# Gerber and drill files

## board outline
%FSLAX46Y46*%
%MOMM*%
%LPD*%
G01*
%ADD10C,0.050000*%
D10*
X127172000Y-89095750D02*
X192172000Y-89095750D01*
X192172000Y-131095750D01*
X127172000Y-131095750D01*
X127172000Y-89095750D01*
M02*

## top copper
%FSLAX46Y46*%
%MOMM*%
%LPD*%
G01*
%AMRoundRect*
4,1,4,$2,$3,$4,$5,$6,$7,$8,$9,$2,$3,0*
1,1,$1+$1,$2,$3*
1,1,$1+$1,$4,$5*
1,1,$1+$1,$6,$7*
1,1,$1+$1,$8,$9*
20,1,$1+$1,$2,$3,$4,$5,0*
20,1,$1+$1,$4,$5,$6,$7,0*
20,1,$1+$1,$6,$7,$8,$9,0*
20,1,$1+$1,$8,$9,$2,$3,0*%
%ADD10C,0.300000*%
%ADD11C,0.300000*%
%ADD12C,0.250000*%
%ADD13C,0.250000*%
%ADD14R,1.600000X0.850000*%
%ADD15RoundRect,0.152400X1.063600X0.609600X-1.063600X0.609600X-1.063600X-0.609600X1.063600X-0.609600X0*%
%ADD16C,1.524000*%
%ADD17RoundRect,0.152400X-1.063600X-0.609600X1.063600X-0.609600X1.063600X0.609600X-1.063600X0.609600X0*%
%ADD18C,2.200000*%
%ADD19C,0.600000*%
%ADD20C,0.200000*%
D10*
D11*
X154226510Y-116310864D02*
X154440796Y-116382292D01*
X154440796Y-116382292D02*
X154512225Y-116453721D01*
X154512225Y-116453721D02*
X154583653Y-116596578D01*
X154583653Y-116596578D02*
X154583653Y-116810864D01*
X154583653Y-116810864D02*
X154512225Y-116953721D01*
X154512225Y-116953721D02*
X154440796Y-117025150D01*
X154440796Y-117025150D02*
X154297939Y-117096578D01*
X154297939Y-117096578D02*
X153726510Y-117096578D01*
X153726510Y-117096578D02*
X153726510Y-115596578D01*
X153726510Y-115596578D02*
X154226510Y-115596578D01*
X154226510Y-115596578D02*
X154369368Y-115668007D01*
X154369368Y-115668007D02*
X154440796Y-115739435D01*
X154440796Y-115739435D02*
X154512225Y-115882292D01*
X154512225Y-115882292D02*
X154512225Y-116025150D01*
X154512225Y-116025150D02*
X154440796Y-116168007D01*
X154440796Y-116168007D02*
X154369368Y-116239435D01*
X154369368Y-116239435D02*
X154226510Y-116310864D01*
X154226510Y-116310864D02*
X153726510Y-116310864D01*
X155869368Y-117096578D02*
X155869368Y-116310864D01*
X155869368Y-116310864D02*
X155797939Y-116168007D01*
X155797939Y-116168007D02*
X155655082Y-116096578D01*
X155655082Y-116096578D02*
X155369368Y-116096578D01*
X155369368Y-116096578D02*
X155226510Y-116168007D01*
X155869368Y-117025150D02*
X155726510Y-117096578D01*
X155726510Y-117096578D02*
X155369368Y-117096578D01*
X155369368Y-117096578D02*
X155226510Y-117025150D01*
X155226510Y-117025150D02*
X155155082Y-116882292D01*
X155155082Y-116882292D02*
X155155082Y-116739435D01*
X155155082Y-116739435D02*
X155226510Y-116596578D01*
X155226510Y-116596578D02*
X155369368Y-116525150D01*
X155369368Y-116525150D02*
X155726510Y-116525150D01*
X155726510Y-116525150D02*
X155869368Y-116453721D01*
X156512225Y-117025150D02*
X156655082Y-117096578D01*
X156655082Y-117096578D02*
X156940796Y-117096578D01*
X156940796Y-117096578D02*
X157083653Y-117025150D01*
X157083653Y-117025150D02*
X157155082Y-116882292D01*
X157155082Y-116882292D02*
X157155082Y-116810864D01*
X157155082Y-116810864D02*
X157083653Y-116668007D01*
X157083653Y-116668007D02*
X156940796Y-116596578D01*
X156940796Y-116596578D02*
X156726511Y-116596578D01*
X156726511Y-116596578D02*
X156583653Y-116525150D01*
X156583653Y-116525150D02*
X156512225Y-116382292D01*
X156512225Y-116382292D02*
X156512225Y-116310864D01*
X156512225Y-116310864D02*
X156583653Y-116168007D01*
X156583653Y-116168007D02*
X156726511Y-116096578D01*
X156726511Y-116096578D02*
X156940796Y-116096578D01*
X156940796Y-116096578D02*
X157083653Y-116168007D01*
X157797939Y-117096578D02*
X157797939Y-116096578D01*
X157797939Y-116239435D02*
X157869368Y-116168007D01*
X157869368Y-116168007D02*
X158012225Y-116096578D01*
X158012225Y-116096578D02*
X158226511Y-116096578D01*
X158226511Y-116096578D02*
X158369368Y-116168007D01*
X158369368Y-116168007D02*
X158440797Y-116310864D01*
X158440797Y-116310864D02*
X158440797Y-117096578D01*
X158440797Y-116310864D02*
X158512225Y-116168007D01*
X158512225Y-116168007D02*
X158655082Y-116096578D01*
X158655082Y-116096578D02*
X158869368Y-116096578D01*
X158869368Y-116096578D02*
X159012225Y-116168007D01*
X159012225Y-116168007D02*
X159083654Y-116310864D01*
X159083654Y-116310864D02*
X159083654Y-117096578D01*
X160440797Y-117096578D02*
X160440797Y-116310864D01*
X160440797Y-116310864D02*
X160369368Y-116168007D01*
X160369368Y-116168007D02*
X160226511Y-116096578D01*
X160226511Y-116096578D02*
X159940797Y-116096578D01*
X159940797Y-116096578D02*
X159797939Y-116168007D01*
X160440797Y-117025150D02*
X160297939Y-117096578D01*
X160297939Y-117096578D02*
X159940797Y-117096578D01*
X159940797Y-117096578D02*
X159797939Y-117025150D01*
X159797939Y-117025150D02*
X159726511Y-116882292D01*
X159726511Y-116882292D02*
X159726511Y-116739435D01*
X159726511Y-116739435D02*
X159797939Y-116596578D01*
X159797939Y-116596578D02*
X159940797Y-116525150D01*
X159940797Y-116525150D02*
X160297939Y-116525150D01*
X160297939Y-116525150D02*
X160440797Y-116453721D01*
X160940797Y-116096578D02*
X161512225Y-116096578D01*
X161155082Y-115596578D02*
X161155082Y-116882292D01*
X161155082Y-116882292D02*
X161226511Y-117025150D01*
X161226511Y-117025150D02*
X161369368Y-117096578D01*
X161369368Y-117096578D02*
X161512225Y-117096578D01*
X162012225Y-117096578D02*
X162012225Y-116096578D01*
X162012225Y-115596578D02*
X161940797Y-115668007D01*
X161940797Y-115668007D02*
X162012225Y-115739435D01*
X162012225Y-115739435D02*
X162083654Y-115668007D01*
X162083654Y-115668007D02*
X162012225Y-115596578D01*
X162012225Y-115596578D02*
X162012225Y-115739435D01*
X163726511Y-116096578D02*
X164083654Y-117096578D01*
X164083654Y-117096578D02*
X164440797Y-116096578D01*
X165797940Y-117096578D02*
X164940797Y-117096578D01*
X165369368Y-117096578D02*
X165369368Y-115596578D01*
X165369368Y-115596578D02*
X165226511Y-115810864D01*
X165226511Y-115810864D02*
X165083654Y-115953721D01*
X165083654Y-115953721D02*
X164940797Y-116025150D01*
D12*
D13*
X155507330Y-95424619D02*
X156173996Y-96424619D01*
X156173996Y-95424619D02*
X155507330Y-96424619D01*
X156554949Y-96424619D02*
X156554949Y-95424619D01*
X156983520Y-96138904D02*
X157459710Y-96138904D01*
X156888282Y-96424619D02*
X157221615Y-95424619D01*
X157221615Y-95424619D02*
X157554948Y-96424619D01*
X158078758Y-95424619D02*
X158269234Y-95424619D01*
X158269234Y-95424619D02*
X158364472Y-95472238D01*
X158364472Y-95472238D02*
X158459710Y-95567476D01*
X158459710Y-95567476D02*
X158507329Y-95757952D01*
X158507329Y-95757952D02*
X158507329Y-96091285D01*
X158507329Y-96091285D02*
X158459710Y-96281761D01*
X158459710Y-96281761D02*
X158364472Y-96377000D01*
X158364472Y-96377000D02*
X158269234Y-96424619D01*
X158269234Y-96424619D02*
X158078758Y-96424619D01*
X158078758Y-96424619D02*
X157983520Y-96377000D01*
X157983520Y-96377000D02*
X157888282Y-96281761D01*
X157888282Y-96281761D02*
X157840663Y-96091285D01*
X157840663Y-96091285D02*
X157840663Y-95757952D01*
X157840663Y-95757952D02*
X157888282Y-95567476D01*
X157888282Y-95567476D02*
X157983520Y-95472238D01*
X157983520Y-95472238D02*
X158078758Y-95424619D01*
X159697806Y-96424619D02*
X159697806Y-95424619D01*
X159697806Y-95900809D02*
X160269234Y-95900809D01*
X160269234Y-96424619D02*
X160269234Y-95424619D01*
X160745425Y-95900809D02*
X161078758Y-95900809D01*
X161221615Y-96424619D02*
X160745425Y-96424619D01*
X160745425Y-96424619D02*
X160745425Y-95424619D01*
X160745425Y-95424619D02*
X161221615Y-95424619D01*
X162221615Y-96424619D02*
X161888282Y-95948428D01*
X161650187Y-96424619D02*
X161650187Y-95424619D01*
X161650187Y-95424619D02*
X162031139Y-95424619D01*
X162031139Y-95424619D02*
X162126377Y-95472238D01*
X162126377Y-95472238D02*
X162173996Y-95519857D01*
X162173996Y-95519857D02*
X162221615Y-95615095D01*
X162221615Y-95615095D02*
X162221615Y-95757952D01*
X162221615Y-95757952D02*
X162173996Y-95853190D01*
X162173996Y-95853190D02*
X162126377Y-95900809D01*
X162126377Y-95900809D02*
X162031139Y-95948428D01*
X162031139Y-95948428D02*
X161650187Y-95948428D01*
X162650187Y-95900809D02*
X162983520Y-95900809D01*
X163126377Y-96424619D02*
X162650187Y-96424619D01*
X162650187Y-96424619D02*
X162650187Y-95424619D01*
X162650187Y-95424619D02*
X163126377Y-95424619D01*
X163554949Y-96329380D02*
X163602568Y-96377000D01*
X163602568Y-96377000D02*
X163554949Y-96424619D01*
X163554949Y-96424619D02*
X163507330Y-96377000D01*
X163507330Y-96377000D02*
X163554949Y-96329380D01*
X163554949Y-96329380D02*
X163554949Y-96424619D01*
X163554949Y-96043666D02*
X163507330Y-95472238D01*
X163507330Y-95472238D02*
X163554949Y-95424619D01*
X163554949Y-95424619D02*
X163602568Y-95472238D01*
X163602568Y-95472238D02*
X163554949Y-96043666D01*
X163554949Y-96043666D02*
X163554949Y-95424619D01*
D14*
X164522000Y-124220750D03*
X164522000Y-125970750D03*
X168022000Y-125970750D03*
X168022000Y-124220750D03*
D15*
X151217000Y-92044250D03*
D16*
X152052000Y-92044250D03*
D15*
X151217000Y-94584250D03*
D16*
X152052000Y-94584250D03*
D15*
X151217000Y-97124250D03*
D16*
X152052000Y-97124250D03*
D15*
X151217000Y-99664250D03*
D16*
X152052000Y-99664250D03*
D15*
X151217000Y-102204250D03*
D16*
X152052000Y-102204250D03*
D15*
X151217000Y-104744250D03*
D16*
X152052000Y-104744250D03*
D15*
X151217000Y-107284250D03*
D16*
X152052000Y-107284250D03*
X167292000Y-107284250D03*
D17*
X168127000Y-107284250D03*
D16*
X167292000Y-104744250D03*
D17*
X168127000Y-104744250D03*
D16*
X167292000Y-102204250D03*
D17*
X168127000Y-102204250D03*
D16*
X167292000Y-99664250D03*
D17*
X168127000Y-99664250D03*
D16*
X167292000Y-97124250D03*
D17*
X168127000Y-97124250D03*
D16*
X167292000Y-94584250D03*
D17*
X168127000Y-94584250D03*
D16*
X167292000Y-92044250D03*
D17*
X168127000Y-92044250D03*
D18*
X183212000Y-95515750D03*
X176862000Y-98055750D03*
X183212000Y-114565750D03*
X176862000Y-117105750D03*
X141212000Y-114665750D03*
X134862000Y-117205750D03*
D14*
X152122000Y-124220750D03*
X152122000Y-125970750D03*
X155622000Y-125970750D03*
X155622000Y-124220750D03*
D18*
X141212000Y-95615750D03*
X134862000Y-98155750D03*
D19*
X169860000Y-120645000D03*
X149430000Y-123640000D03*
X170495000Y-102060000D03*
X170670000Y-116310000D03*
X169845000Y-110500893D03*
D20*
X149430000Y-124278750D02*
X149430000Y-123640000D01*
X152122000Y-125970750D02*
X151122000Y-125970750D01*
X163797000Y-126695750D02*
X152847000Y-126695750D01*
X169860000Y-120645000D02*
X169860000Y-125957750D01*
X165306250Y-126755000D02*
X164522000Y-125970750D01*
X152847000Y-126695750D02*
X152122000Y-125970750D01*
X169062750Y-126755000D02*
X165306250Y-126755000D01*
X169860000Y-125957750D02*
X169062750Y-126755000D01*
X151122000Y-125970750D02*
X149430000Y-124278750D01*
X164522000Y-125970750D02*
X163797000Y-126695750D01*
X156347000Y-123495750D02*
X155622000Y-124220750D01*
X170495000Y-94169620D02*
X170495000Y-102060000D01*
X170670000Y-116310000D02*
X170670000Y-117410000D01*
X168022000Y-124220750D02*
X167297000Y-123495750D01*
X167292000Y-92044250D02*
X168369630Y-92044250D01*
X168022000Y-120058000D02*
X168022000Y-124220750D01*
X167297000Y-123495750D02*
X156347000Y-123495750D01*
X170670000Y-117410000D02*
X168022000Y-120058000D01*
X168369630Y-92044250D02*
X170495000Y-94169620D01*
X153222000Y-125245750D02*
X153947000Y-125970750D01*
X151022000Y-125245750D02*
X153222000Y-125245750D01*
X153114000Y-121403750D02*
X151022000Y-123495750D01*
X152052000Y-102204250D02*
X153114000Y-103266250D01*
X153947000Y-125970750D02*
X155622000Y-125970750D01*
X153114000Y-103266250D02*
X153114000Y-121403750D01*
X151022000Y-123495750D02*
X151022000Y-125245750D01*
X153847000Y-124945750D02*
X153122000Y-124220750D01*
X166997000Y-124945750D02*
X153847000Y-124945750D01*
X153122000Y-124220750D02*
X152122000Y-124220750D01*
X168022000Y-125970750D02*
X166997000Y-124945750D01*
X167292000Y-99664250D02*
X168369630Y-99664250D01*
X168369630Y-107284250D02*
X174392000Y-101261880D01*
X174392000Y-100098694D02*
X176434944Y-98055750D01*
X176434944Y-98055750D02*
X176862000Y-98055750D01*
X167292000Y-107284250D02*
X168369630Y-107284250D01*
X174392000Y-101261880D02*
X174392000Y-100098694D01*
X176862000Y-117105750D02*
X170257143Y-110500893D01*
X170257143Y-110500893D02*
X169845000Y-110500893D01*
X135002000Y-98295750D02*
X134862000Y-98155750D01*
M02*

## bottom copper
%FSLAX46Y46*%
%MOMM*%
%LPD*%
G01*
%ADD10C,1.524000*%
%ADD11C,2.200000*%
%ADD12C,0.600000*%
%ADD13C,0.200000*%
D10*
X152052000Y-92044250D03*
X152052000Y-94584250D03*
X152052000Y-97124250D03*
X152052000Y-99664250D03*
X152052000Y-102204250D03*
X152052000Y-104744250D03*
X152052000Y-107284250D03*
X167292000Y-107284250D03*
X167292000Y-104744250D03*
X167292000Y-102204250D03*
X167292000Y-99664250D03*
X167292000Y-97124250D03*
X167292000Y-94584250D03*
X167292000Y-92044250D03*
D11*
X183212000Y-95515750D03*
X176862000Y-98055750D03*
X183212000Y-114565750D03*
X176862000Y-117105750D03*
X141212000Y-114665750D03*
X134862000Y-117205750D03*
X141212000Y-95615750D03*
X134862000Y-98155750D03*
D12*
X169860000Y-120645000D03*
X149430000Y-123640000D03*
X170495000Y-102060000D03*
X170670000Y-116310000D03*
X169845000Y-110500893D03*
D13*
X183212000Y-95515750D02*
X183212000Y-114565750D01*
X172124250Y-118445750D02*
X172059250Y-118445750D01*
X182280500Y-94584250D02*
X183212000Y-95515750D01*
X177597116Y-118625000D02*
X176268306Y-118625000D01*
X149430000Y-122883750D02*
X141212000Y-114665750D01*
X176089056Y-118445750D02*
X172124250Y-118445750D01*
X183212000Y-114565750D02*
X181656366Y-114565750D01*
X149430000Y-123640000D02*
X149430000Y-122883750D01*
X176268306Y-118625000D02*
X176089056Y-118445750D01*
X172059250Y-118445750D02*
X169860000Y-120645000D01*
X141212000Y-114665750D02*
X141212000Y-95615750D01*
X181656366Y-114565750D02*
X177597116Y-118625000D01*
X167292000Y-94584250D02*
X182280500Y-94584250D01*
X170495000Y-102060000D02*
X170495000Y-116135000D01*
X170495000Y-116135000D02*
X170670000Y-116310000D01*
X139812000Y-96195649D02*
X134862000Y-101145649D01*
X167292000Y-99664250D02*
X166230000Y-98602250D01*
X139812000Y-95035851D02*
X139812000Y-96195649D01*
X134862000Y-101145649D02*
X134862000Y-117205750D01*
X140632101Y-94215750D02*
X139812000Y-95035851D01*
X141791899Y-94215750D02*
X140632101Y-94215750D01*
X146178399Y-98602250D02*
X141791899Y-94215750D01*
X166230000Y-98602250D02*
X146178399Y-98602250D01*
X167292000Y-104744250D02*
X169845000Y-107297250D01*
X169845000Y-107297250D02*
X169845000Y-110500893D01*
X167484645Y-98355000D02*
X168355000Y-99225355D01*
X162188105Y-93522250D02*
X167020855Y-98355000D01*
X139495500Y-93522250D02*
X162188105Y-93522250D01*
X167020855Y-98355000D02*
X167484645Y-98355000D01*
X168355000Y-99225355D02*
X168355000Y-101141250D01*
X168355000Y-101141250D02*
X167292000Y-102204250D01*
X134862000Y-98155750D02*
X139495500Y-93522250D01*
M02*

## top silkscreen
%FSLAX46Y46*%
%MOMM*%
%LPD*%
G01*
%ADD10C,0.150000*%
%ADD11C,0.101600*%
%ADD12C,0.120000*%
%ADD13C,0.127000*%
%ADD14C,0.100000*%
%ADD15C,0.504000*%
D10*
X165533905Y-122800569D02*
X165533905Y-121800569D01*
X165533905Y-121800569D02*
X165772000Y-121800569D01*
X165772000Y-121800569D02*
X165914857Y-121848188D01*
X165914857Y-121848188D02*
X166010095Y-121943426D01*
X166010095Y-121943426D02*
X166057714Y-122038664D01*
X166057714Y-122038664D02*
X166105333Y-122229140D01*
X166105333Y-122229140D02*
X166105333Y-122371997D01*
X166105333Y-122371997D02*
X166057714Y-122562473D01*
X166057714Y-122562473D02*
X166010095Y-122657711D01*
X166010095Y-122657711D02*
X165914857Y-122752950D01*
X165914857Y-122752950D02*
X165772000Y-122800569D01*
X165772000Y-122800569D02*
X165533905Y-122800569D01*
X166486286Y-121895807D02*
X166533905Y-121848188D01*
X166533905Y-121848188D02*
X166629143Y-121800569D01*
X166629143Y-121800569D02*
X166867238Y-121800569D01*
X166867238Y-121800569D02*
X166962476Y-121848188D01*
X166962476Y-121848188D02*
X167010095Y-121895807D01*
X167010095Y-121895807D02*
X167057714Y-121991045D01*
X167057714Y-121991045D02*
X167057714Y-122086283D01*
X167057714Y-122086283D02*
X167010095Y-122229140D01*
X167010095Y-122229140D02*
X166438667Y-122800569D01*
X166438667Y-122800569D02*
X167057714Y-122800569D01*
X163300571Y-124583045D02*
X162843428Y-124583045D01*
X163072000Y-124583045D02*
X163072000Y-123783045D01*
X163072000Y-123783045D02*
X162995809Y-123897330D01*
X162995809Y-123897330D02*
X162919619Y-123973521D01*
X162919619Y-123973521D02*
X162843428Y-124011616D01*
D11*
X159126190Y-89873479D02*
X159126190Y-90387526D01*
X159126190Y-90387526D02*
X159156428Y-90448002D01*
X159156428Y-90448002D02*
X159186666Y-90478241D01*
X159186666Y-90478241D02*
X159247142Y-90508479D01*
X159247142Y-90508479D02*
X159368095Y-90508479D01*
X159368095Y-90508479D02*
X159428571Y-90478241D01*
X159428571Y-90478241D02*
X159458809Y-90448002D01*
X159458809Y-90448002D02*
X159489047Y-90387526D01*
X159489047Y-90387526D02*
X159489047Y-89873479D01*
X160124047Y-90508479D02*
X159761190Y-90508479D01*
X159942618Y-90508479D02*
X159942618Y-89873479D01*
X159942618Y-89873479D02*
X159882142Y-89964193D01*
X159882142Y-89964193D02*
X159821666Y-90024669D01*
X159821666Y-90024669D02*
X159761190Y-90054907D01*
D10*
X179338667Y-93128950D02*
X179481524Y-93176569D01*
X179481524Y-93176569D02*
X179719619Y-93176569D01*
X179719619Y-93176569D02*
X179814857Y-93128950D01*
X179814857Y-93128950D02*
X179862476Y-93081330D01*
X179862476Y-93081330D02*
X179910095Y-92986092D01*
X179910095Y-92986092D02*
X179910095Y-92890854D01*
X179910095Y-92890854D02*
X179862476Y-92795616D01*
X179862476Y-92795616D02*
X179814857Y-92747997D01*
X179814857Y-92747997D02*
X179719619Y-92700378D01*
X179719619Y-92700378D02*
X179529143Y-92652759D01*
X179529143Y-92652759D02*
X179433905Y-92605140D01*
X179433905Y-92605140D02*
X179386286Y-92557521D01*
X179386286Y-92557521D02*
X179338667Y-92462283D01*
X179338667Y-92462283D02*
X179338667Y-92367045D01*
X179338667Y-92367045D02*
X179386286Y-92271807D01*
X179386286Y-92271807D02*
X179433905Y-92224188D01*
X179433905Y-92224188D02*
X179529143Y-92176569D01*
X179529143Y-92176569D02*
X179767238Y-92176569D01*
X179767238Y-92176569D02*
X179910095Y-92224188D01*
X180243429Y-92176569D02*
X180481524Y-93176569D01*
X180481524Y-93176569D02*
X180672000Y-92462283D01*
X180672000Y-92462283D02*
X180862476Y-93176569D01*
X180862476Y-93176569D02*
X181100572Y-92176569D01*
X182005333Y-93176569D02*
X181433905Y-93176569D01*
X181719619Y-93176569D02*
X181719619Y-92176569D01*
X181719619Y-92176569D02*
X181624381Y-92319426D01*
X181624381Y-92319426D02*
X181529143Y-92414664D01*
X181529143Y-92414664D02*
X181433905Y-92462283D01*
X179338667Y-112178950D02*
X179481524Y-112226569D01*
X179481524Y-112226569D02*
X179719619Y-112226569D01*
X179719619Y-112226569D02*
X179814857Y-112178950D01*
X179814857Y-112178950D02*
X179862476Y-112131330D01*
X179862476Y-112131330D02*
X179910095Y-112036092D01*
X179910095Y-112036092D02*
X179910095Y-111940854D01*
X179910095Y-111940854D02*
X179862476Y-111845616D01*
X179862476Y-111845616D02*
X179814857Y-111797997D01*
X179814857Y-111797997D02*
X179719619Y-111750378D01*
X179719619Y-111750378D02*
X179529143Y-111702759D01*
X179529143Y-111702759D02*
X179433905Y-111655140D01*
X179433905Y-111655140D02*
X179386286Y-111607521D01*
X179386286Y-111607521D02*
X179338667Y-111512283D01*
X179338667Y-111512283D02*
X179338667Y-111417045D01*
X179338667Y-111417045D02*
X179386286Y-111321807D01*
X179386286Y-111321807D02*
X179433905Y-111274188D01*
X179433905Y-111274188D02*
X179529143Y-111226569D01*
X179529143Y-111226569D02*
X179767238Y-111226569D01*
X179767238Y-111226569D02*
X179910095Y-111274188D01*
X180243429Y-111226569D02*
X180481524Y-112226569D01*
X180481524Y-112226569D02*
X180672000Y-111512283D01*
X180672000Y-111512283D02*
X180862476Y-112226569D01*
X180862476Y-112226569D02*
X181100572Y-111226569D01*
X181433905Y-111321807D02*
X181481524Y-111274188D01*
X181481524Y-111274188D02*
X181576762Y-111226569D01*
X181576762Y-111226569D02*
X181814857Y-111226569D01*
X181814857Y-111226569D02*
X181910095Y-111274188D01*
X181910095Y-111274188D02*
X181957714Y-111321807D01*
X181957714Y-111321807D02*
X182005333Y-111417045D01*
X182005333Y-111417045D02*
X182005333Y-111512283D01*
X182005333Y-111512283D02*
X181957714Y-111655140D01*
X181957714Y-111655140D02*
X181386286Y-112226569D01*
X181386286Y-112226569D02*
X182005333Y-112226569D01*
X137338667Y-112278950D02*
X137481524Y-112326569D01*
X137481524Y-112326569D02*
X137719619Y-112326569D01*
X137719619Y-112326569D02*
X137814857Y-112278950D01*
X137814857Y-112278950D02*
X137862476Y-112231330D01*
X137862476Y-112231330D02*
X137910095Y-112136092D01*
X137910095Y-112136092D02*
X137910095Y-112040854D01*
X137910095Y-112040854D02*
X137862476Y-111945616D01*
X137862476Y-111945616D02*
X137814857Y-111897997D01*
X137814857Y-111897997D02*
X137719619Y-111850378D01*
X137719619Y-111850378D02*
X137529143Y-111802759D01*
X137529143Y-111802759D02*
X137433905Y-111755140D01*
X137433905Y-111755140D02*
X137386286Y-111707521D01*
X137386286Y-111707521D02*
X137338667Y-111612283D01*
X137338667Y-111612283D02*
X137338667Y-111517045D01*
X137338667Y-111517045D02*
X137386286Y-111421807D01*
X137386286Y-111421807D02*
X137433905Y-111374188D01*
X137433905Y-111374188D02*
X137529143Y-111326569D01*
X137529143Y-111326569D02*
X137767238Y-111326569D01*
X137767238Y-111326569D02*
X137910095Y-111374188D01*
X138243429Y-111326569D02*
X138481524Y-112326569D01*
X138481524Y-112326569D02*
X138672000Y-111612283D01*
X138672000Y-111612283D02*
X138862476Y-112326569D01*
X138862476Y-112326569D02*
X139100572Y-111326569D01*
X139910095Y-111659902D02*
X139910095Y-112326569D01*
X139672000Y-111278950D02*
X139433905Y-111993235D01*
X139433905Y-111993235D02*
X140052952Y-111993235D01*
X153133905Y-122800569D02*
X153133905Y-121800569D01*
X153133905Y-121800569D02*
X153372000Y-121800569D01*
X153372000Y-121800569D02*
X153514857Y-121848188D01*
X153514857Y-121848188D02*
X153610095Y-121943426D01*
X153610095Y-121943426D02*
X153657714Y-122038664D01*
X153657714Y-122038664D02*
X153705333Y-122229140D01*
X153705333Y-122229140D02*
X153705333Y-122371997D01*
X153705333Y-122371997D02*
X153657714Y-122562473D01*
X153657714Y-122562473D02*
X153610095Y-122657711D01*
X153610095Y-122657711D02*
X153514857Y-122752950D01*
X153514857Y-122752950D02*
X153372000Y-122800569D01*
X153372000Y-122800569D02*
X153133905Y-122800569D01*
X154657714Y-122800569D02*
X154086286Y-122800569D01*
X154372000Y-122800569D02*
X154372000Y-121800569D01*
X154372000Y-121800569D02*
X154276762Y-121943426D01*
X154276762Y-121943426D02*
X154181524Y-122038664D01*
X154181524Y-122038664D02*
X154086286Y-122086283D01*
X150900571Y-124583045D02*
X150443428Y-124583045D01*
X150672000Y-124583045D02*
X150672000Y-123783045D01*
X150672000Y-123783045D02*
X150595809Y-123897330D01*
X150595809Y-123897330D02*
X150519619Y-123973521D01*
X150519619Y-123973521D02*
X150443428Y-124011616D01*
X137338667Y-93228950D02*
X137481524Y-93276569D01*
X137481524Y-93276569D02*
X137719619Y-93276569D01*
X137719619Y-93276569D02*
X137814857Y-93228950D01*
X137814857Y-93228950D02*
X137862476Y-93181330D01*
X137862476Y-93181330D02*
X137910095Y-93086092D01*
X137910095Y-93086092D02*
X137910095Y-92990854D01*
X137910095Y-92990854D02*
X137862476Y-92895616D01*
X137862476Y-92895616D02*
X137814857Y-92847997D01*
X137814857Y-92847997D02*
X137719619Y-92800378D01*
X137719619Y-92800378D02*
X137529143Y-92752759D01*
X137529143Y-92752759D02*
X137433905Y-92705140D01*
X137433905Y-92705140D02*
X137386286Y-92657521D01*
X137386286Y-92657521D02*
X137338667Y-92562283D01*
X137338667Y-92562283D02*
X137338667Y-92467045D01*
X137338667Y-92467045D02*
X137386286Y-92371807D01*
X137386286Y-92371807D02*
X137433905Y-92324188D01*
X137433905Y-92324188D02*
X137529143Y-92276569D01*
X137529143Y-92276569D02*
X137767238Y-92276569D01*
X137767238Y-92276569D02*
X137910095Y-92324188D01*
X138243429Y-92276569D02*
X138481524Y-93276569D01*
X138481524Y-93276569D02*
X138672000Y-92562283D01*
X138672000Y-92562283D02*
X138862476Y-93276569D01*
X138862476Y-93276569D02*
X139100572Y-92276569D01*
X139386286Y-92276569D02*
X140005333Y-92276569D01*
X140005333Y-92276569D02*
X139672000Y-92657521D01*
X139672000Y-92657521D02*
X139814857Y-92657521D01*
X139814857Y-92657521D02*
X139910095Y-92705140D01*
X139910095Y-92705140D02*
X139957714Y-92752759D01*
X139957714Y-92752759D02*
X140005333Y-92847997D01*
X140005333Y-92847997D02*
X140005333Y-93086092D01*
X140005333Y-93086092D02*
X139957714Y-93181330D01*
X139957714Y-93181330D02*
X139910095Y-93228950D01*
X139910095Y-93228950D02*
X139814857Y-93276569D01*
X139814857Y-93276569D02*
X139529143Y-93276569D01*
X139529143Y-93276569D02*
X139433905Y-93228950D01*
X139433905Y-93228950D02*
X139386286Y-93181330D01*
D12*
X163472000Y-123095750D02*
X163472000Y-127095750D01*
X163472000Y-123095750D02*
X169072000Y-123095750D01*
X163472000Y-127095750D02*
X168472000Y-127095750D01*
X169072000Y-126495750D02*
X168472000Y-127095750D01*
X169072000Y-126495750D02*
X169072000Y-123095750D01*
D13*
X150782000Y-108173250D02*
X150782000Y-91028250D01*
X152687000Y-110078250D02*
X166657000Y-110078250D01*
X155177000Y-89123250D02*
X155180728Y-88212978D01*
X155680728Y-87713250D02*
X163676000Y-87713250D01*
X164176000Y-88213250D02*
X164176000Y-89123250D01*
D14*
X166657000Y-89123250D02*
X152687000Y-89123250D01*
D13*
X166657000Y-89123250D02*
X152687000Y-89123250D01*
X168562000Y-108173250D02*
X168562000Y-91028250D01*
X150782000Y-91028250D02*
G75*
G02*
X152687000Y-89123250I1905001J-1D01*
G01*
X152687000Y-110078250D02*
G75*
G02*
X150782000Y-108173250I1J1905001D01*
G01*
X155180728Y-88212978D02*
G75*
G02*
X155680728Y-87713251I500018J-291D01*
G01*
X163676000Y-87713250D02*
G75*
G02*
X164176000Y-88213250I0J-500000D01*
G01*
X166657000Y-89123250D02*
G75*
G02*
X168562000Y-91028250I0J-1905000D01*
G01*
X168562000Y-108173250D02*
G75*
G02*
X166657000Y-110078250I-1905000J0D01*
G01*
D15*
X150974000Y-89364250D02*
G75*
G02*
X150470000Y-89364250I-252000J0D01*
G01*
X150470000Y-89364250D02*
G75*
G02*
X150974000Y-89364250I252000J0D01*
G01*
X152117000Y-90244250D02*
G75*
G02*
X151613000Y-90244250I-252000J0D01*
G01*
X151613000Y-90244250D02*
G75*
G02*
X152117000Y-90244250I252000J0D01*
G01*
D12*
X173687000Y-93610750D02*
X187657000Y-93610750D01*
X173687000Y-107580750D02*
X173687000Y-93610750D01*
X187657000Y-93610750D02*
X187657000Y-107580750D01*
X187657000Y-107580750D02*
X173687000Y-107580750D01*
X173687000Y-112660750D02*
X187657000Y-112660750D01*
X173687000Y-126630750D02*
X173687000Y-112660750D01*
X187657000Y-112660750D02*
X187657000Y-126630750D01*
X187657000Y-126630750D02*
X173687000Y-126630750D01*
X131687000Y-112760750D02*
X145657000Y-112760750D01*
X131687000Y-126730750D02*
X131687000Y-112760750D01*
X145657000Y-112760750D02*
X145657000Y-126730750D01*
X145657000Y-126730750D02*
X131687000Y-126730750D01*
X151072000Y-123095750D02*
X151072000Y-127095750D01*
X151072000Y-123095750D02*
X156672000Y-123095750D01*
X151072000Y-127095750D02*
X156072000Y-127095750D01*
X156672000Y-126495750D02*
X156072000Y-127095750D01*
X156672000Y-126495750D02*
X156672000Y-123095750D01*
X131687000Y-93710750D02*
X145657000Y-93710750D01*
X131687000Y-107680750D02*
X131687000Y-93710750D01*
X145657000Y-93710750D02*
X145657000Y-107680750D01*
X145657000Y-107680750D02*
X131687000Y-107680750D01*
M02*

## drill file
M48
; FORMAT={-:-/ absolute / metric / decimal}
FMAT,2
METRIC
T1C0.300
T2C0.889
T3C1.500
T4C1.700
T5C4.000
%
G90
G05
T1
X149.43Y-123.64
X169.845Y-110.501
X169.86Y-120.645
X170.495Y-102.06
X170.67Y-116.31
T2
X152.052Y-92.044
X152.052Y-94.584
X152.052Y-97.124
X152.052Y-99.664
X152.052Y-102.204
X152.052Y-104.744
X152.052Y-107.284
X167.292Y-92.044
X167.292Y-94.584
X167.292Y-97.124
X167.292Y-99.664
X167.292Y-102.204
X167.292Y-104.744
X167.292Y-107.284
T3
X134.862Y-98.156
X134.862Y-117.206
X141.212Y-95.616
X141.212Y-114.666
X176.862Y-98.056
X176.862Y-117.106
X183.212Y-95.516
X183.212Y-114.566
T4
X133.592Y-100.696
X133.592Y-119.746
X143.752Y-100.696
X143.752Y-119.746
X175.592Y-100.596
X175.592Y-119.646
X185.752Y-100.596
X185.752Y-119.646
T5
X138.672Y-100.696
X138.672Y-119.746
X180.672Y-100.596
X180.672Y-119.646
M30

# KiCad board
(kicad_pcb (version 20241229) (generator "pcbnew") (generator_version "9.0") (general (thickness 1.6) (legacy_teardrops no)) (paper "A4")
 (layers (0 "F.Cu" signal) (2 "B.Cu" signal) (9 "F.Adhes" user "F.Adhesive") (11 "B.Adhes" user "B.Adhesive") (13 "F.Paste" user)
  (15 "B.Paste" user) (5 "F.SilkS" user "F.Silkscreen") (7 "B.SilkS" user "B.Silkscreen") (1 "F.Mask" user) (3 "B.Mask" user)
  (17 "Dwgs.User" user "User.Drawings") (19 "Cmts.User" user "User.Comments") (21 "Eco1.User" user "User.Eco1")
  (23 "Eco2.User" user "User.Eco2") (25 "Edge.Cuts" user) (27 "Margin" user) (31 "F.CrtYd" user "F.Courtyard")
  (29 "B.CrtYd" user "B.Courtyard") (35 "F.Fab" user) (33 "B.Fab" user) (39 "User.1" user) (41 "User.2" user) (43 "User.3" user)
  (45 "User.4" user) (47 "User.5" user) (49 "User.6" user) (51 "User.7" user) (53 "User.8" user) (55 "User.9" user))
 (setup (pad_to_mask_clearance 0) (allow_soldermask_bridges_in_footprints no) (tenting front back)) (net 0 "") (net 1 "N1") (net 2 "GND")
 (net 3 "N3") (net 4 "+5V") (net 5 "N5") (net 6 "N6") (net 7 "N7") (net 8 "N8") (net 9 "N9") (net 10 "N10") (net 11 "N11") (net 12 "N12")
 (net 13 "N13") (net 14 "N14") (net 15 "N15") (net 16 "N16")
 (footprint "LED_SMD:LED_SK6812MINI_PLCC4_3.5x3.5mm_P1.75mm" (layer "F.Cu") (at 166.272 125.09575)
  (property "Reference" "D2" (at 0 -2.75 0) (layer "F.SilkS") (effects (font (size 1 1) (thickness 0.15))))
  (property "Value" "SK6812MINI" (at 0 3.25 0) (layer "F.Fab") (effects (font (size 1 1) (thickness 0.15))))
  (fp_line (start -2.8 -2) (end -2.8 2) (stroke (width 0.12) (type default)) (layer "F.SilkS"))
  (fp_line (start -2.8 -2) (end 2.8 -2) (stroke (width 0.12) (type solid)) (layer "F.SilkS"))
  (fp_line (start -2.8 2) (end 2.2 2) (stroke (width 0.12) (type solid)) (layer "F.SilkS"))
  (fp_line (start 2.8 1.4) (end 2.2 2) (stroke (width 0.12) (type default)) (layer "F.SilkS"))
  (fp_line (start 2.8 1.4) (end 2.8 -2) (stroke (width 0.12) (type solid)) (layer "F.SilkS"))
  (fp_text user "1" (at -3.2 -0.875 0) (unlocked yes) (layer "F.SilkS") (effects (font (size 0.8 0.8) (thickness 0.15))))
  (pad "1" smd rect (at -1.75 -0.875) (size 1.6 0.85) (layers "F.Cu" "F.Mask" "F.Paste") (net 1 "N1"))
  (pad "2" smd rect (at -1.75 0.875) (size 1.6 0.85) (layers "F.Cu" "F.Mask" "F.Paste") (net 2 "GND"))
  (pad "3" smd rect (at 1.75 0.875) (size 1.6 0.85) (layers "F.Cu" "F.Mask" "F.Paste") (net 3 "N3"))
  (pad "4" smd rect (at 1.75 -0.875) (size 1.6 0.85) (layers "F.Cu" "F.Mask" "F.Paste") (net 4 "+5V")))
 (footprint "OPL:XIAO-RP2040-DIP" (layer "F.Cu") (at 159.672 99.66425)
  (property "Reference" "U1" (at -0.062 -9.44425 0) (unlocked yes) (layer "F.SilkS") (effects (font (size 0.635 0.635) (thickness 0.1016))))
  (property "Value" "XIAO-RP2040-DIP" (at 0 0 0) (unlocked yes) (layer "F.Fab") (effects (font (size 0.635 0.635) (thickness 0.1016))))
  (fp_line (start -8.89 8.509) (end -8.89 -8.636) (stroke (width 0.127) (type solid)) (layer "F.SilkS"))
  (fp_line (start -6.985 10.414) (end 6.985 10.414) (stroke (width 0.127) (type solid)) (layer "F.SilkS"))
  (fp_line (start -4.495 -10.541) (end -4.491272 -11.451272) (stroke (width 0.127) (type solid)) (layer "F.SilkS"))
  (fp_line (start -3.991272 -11.951) (end 4.004 -11.951) (stroke (width 0.127) (type solid)) (layer "F.SilkS"))
  (fp_line (start 4.504 -11.451) (end 4.504 -10.541) (stroke (width 0.127) (type solid)) (layer "F.SilkS"))
  (fp_line (start 6.985 -10.541) (end -6.985 -10.541) (stroke (width 0.1) (type solid)) (layer "F.SilkS"))
  (fp_line (start 6.985 -10.541) (end -6.985 -10.541) (stroke (width 0.127) (type solid)) (layer "F.SilkS"))
  (fp_line (start 8.89 8.509) (end 8.89 -8.636) (stroke (width 0.127) (type solid)) (layer "F.SilkS"))
  (fp_arc (start -8.89 -8.636) (mid -8.332038 -9.983038) (end -6.985 -10.541) (stroke (width 0.127) (type solid)) (layer "F.SilkS"))
  (fp_arc (start -6.985 10.414) (mid -8.332038 9.856038) (end -8.89 8.509) (stroke (width 0.127) (type solid)) (layer "F.SilkS"))
  (fp_arc (start -4.491272 -11.451272) (mid -4.344724 -11.804644) (end -3.991272 -11.951) (stroke (width 0.127) (type default))
   (layer "F.SilkS"))
  (fp_arc (start 4.004 -11.951) (mid 4.357553 -11.804553) (end 4.504 -11.451) (stroke (width 0.127) (type default)) (layer "F.SilkS"))
  (fp_arc (start 6.985 -10.541) (mid 8.332038 -9.983038) (end 8.89 -8.636) (stroke (width 0.127) (type solid)) (layer "F.SilkS"))
  (fp_arc (start 8.89 8.509) (mid 8.332038 9.856038) (end 6.985 10.414) (stroke (width 0.127) (type solid)) (layer "F.SilkS"))
  (fp_circle (center -8.95 -10.3) (end -8.95 -10.554) (stroke (width 0.5) (type solid)) (fill yes) (layer "F.SilkS"))
  (fp_circle (center -7.807 -9.42) (end -7.807 -9.674) (stroke (width 0.5) (type solid)) (fill yes) (layer "F.SilkS"))
  (pad "1" smd roundrect (at -8.455 -7.62 180) (size 2.432 1.524) (layers "F.Cu" "F.Mask") (roundrect_rratio 0.1) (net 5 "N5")
   (thermal_bridge_angle 45))
  (pad "1" thru_hole circle (at -7.62 -7.62 180) (size 1.524 1.524) (drill 0.889) (layers "*.Cu" "*.Mask") (remove_unused_layers no)
   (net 5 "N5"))
  (pad "2" smd roundrect (at -8.455 -5.08 180) (size 2.432 1.524) (layers "F.Cu" "F.Mask") (roundrect_rratio 0.1) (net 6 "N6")
   (thermal_bridge_angle 45))
  (pad "2" thru_hole circle (at -7.62 -5.08 180) (size 1.524 1.524) (drill 0.889) (layers "*.Cu" "*.Mask") (remove_unused_layers no)
   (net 6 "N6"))
  (pad "3" smd roundrect (at -8.455 -2.54 180) (size 2.432 1.524) (layers "F.Cu" "F.Mask") (roundrect_rratio 0.1) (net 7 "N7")
   (thermal_bridge_angle 45))
  (pad "3" thru_hole circle (at -7.62 -2.54 180) (size 1.524 1.524) (drill 0.889) (layers "*.Cu" "*.Mask") (remove_unused_layers no)
   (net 7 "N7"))
  (pad "4" smd roundrect (at -8.455 0 180) (size 2.432 1.524) (layers "F.Cu" "F.Mask") (roundrect_rratio 0.1) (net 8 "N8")
   (thermal_bridge_angle 45))
  (pad "4" thru_hole circle (at -7.62 0 180) (size 1.524 1.524) (drill 0.889) (layers "*.Cu" "*.Mask") (remove_unused_layers no)
   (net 8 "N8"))
  (pad "5" smd roundrect (at -8.455 2.54 180) (size 2.432 1.524) (layers "F.Cu" "F.Mask") (roundrect_rratio 0.1) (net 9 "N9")
   (thermal_bridge_angle 45))
  (pad "5" thru_hole circle (at -7.62 2.54 180) (size 1.524 1.524) (drill 0.889) (layers "*.Cu" "*.Mask") (remove_unused_layers no)
   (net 9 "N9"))
  (pad "6" smd roundrect (at -8.455 5.08 180) (size 2.432 1.524) (layers "F.Cu" "F.Mask") (roundrect_rratio 0.1) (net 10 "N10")
   (thermal_bridge_angle 45))
  (pad "6" thru_hole circle (at -7.62 5.08 180) (size 1.524 1.524) (drill 0.889) (layers "*.Cu" "*.Mask") (remove_unused_layers no)
   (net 10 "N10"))
  (pad "7" smd roundrect (at -8.455 7.62 180) (size 2.432 1.524) (layers "F.Cu" "F.Mask") (roundrect_rratio 0.1) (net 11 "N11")
   (thermal_bridge_angle 45))
  (pad "7" thru_hole circle (at -7.62 7.62 180) (size 1.524 1.524) (drill 0.889) (layers "*.Cu" "*.Mask") (remove_unused_layers no)
   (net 11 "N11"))
  (pad "8" thru_hole circle (at 7.62 7.62) (size 1.524 1.524) (drill 0.889) (layers "*.Cu" "*.Mask") (remove_unused_layers no)
   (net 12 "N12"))
  (pad "8" smd roundrect (at 8.455 7.62) (size 2.432 1.524) (layers "F.Cu" "F.Mask") (roundrect_rratio 0.1) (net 12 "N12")
   (thermal_bridge_angle 45))
  (pad "9" thru_hole circle (at 7.62 5.08) (size 1.524 1.524) (drill 0.889) (layers "*.Cu" "*.Mask") (remove_unused_layers no)
   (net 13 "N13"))
  (pad "9" smd roundrect (at 8.455 5.08) (size 2.432 1.524) (layers "F.Cu" "F.Mask") (roundrect_rratio 0.1) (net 13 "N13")
   (thermal_bridge_angle 45))
  (pad "10" thru_hole circle (at 7.62 2.54) (size 1.524 1.524) (drill 0.889) (layers "*.Cu" "*.Mask") (remove_unused_layers no)
   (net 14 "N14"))
  (pad "10" smd roundrect (at 8.455 2.54) (size 2.432 1.524) (layers "F.Cu" "F.Mask") (roundrect_rratio 0.1) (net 14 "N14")
   (thermal_bridge_angle 45))
  (pad "11" thru_hole circle (at 7.62 0) (size 1.524 1.524) (drill 0.889) (layers "*.Cu" "*.Mask") (remove_unused_layers no) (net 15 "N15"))
  (pad "11" smd roundrect (at 8.455 0) (size 2.432 1.524) (layers "F.Cu" "F.Mask") (roundrect_rratio 0.1) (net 15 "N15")
   (thermal_bridge_angle 45))
  (pad "12" thru_hole circle (at 7.62 -2.54) (size 1.524 1.524) (drill 0.889) (layers "*.Cu" "*.Mask") (remove_unused_layers no)
   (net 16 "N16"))
  (pad "12" smd roundrect (at 8.455 -2.54) (size 2.432 1.524) (layers "F.Cu" "F.Mask") (roundrect_rratio 0.1) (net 16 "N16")
   (thermal_bridge_angle 45))
  (pad "13" thru_hole circle (at 7.62 -5.08) (size 1.524 1.524) (drill 0.889) (layers "*.Cu" "*.Mask") (remove_unused_layers no)
   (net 2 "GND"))
  (pad "13" smd roundrect (at 8.455 -5.08) (size 2.432 1.524) (layers "F.Cu" "F.Mask") (roundrect_rratio 0.1) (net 2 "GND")
   (thermal_bridge_angle 45))
  (pad "14" thru_hole circle (at 7.62 -7.62) (size 1.524 1.524) (drill 0.889) (layers "*.Cu" "*.Mask") (remove_unused_layers no)
   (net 4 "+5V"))
  (pad "14" smd roundrect (at 8.455 -7.62) (size 2.432 1.524) (layers "F.Cu" "F.Mask") (roundrect_rratio 0.1) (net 4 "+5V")
   (thermal_bridge_angle 45)))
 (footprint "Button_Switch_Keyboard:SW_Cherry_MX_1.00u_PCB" (layer "F.Cu") (at 183.212 95.51575)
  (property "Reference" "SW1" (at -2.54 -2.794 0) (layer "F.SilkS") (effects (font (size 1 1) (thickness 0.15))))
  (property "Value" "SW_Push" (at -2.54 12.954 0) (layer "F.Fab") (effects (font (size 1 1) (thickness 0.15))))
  (fp_line (start -9.525 -1.905) (end 4.445 -1.905) (stroke (width 0.12) (type solid)) (layer "F.SilkS"))
  (fp_line (start -9.525 12.065) (end -9.525 -1.905) (stroke (width 0.12) (type solid)) (layer "F.SilkS"))
  (fp_line (start 4.445 -1.905) (end 4.445 12.065) (stroke (width 0.12) (type solid)) (layer "F.SilkS"))
  (fp_line (start 4.445 12.065) (end -9.525 12.065) (stroke (width 0.12) (type solid)) (layer "F.SilkS"))
  (pad "" np_thru_hole circle (at -7.62 5.08) (size 1.7 1.7) (drill 1.7) (layers "*.Cu" "*.Mask"))
  (pad "" np_thru_hole circle (at -2.54 5.08) (size 4 4) (drill 4) (layers "*.Cu" "*.Mask"))
  (pad "" np_thru_hole circle (at 2.54 5.08) (size 1.7 1.7) (drill 1.7) (layers "*.Cu" "*.Mask"))
  (pad "1" thru_hole circle (at 0 0) (size 2.2 2.2) (drill 1.5) (layers "*.Cu" "*.Mask") (remove_unused_layers no) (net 2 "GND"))
  (pad "2" thru_hole circle (at -6.35 2.54) (size 2.2 2.2) (drill 1.5) (layers "*.Cu" "*.Mask") (remove_unused_layers no) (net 12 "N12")))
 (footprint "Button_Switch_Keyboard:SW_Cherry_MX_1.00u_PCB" (layer "F.Cu") (at 183.212 114.56575)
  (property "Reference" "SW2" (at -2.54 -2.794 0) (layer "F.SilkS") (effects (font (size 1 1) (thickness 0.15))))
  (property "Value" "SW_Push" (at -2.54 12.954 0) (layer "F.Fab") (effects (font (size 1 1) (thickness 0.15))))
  (fp_line (start -9.525 -1.905) (end 4.445 -1.905) (stroke (width 0.12) (type solid)) (layer "F.SilkS"))
  (fp_line (start -9.525 12.065) (end -9.525 -1.905) (stroke (width 0.12) (type solid)) (layer "F.SilkS"))
  (fp_line (start 4.445 -1.905) (end 4.445 12.065) (stroke (width 0.12) (type solid)) (layer "F.SilkS"))
  (fp_line (start 4.445 12.065) (end -9.525 12.065) (stroke (width 0.12) (type solid)) (layer "F.SilkS"))
  (pad "" np_thru_hole circle (at -7.62 5.08) (size 1.7 1.7) (drill 1.7) (layers "*.Cu" "*.Mask"))
  (pad "" np_thru_hole circle (at -2.54 5.08) (size 4 4) (drill 4) (layers "*.Cu" "*.Mask"))
  (pad "" np_thru_hole circle (at 2.54 5.08) (size 1.7 1.7) (drill 1.7) (layers "*.Cu" "*.Mask"))
  (pad "1" thru_hole circle (at 0 0) (size 2.2 2.2) (drill 1.5) (layers "*.Cu" "*.Mask") (remove_unused_layers no) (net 2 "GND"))
  (pad "2" thru_hole circle (at -6.35 2.54) (size 2.2 2.2) (drill 1.5) (layers "*.Cu" "*.Mask") (remove_unused_layers no) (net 13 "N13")))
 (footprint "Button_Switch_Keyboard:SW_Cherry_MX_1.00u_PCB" (layer "F.Cu") (at 141.212 114.66575)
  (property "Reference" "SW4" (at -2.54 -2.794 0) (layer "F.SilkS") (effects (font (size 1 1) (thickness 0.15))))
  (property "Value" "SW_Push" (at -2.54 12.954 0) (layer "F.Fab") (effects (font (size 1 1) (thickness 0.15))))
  (fp_line (start -9.525 -1.905) (end 4.445 -1.905) (stroke (width 0.12) (type solid)) (layer "F.SilkS"))
  (fp_line (start -9.525 12.065) (end -9.525 -1.905) (stroke (width 0.12) (type solid)) (layer "F.SilkS"))
  (fp_line (start 4.445 -1.905) (end 4.445 12.065) (stroke (width 0.12) (type solid)) (layer "F.SilkS"))
  (fp_line (start 4.445 12.065) (end -9.525 12.065) (stroke (width 0.12) (type solid)) (layer "F.SilkS"))
  (pad "" np_thru_hole circle (at -7.62 5.08) (size 1.7 1.7) (drill 1.7) (layers "*.Cu" "*.Mask"))
  (pad "" np_thru_hole circle (at -2.54 5.08) (size 4 4) (drill 4) (layers "*.Cu" "*.Mask"))
  (pad "" np_thru_hole circle (at 2.54 5.08) (size 1.7 1.7) (drill 1.7) (layers "*.Cu" "*.Mask"))
  (pad "1" thru_hole circle (at 0 0) (size 2.2 2.2) (drill 1.5) (layers "*.Cu" "*.Mask") (remove_unused_layers no) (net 2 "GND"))
  (pad "2" thru_hole circle (at -6.35 2.54) (size 2.2 2.2) (drill 1.5) (layers "*.Cu" "*.Mask") (remove_unused_layers no) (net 15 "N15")))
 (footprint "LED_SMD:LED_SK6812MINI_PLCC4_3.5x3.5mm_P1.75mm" (layer "F.Cu") (at 153.872 125.09575)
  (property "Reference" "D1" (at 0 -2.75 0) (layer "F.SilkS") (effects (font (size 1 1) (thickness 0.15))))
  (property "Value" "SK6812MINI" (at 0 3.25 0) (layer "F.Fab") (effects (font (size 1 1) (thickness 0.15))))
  (fp_line (start -2.8 -2) (end -2.8 2) (stroke (width 0.12) (type default)) (layer "F.SilkS"))
  (fp_line (start -2.8 -2) (end 2.8 -2) (stroke (width 0.12) (type solid)) (layer "F.SilkS"))
  (fp_line (start -2.8 2) (end 2.2 2) (stroke (width 0.12) (type solid)) (layer "F.SilkS"))
  (fp_line (start 2.8 1.4) (end 2.2 2) (stroke (width 0.12) (type default)) (layer "F.SilkS"))
  (fp_line (start 2.8 1.4) (end 2.8 -2) (stroke (width 0.12) (type solid)) (layer "F.SilkS"))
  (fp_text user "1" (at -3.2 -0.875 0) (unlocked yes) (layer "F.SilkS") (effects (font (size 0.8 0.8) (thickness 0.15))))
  (pad "1" smd rect (at -1.75 -0.875) (size 1.6 0.85) (layers "F.Cu" "F.Mask" "F.Paste") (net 3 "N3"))
  (pad "2" smd rect (at -1.75 0.875) (size 1.6 0.85) (layers "F.Cu" "F.Mask" "F.Paste") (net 2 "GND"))
  (pad "3" smd rect (at 1.75 0.875) (size 1.6 0.85) (layers "F.Cu" "F.Mask" "F.Paste") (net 9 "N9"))
  (pad "4" smd rect (at 1.75 -0.875) (size 1.6 0.85) (layers "F.Cu" "F.Mask" "F.Paste") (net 4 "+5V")))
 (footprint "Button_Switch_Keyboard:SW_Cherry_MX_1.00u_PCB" (layer "F.Cu") (at 141.212 95.61575)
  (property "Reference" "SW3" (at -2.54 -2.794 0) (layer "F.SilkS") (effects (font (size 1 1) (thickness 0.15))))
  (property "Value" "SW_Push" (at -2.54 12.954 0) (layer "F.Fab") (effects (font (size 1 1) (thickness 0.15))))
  (fp_line (start -9.525 -1.905) (end 4.445 -1.905) (stroke (width 0.12) (type solid)) (layer "F.SilkS"))
  (fp_line (start -9.525 12.065) (end -9.525 -1.905) (stroke (width 0.12) (type solid)) (layer "F.SilkS"))
  (fp_line (start 4.445 -1.905) (end 4.445 12.065) (stroke (width 0.12) (type solid)) (layer "F.SilkS"))
  (fp_line (start 4.445 12.065) (end -9.525 12.065) (stroke (width 0.12) (type solid)) (layer "F.SilkS"))
  (pad "" np_thru_hole circle (at -7.62 5.08) (size 1.7 1.7) (drill 1.7) (layers "*.Cu" "*.Mask"))
  (pad "" np_thru_hole circle (at -2.54 5.08) (size 4 4) (drill 4) (layers "*.Cu" "*.Mask"))
  (pad "" np_thru_hole circle (at 2.54 5.08) (size 1.7 1.7) (drill 1.7) (layers "*.Cu" "*.Mask"))
  (pad "1" thru_hole circle (at 0 0) (size 2.2 2.2) (drill 1.5) (layers "*.Cu" "*.Mask") (remove_unused_layers no) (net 2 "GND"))
  (pad "2" thru_hole circle (at -6.35 2.54) (size 2.2 2.2) (drill 1.5) (layers "*.Cu" "*.Mask") (remove_unused_layers no) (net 14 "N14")))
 (gr_rect (start 127.172 89.09575) (end 192.172 131.09575) (stroke (width 0.05) (type default)) (fill no) (layer "Edge.Cuts"))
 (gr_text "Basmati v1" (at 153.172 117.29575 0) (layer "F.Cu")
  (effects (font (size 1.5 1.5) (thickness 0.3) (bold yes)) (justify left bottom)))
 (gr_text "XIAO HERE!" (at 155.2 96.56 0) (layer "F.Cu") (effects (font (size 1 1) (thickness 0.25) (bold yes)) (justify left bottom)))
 (segment (start 149.43 124.27875) (end 149.43 123.64) (width 0.2) (layer "F.Cu") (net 2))
 (segment (start 152.122 125.97075) (end 151.122 125.97075) (width 0.2) (layer "F.Cu") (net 2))
 (segment (start 163.797 126.69575) (end 152.847 126.69575) (width 0.2) (layer "F.Cu") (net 2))
 (segment (start 169.86 120.645) (end 169.86 125.95775) (width 0.2) (layer "F.Cu") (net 2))
 (segment (start 165.30625 126.755) (end 164.522 125.97075) (width 0.2) (layer "F.Cu") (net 2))
 (segment (start 152.847 126.69575) (end 152.122 125.97075) (width 0.2) (layer "F.Cu") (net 2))
 (segment (start 169.06275 126.755) (end 165.30625 126.755) (width 0.2) (layer "F.Cu") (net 2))
 (segment (start 169.86 125.95775) (end 169.06275 126.755) (width 0.2) (layer "F.Cu") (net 2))
 (segment (start 151.122 125.97075) (end 149.43 124.27875) (width 0.2) (layer "F.Cu") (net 2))
 (segment (start 164.522 125.97075) (end 163.797 126.69575) (width 0.2) (layer "F.Cu") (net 2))
 (via (at 169.86 120.645) (size 0.6) (drill 0.3) (layers "F.Cu" "B.Cu") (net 2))
 (via (at 149.43 123.64) (size 0.6) (drill 0.3) (layers "F.Cu" "B.Cu") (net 2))
 (segment (start 183.212 95.51575) (end 183.212 114.56575) (width 0.2) (layer "B.Cu") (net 2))
 (segment (start 172.12425 118.44575) (end 172.05925 118.44575) (width 0.2) (layer "B.Cu") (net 2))
 (segment (start 182.2805 94.58425) (end 183.212 95.51575) (width 0.2) (layer "B.Cu") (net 2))
 (segment (start 177.597116 118.625) (end 176.268306 118.625) (width 0.2) (layer "B.Cu") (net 2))
 (segment (start 149.43 122.88375) (end 141.212 114.66575) (width 0.2) (layer "B.Cu") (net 2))
 (segment (start 176.089056 118.44575) (end 172.12425 118.44575) (width 0.2) (layer "B.Cu") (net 2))
 (segment (start 183.212 114.56575) (end 181.656366 114.56575) (width 0.2) (layer "B.Cu") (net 2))
 (segment (start 149.43 123.64) (end 149.43 122.88375) (width 0.2) (layer "B.Cu") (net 2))
 (segment (start 176.268306 118.625) (end 176.089056 118.44575) (width 0.2) (layer "B.Cu") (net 2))
 (segment (start 172.05925 118.44575) (end 169.86 120.645) (width 0.2) (layer "B.Cu") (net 2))
 (segment (start 141.212 114.66575) (end 141.212 95.61575) (width 0.2) (layer "B.Cu") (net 2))
 (segment (start 181.656366 114.56575) (end 177.597116 118.625) (width 0.2) (layer "B.Cu") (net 2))
 (segment (start 167.292 94.58425) (end 182.2805 94.58425) (width 0.2) (layer "B.Cu") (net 2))
 (segment (start 156.347 123.49575) (end 155.622 124.22075) (width 0.2) (layer "F.Cu") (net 4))
 (segment (start 170.495 94.16962) (end 170.495 102.06) (width 0.2) (layer "F.Cu") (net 4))
 (segment (start 170.67 116.31) (end 170.67 117.41) (width 0.2) (layer "F.Cu") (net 4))
 (segment (start 168.022 124.22075) (end 167.297 123.49575) (width 0.2) (layer "F.Cu") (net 4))
 (segment (start 167.292 92.04425) (end 168.36963 92.04425) (width 0.2) (layer "F.Cu") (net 4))
 (segment (start 168.022 120.058) (end 168.022 124.22075) (width 0.2) (layer "F.Cu") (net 4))
 (segment (start 167.297 123.49575) (end 156.347 123.49575) (width 0.2) (layer "F.Cu") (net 4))
 (segment (start 170.67 117.41) (end 168.022 120.058) (width 0.2) (layer "F.Cu") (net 4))
 (segment (start 168.36963 92.04425) (end 170.495 94.16962) (width 0.2) (layer "F.Cu") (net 4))
 (via (at 170.495 102.06) (size 0.6) (drill 0.3) (layers "F.Cu" "B.Cu") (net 4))
 (via (at 170.67 116.31) (size 0.6) (drill 0.3) (layers "F.Cu" "B.Cu") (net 4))
 (segment (start 170.495 102.06) (end 170.495 116.135) (width 0.2) (layer "B.Cu") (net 4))
 (segment (start 170.495 116.135) (end 170.67 116.31) (width 0.2) (layer "B.Cu") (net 4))
 (segment (start 153.222 125.24575) (end 153.947 125.97075) (width 0.2) (layer "F.Cu") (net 9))
 (segment (start 151.022 125.24575) (end 153.222 125.24575) (width 0.2) (layer "F.Cu") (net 9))
 (segment (start 153.114 121.40375) (end 151.022 123.49575) (width 0.2) (layer "F.Cu") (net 9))
 (segment (start 152.052 102.20425) (end 153.114 103.26625) (width 0.2) (layer "F.Cu") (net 9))
 (segment (start 153.947 125.97075) (end 155.622 125.97075) (width 0.2) (layer "F.Cu") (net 9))
 (segment (start 153.114 103.26625) (end 153.114 121.40375) (width 0.2) (layer "F.Cu") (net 9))
 (segment (start 151.022 123.49575) (end 151.022 125.24575) (width 0.2) (layer "F.Cu") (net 9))
 (segment (start 153.847 124.94575) (end 153.122 124.22075) (width 0.2) (layer "F.Cu") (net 3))
 (segment (start 166.997 124.94575) (end 153.847 124.94575) (width 0.2) (layer "F.Cu") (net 3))
 (segment (start 153.122 124.22075) (end 152.122 124.22075) (width 0.2) (layer "F.Cu") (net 3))
 (segment (start 168.022 125.97075) (end 166.997 124.94575) (width 0.2) (layer "F.Cu") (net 3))
 (segment (start 167.292 99.66425) (end 168.36963 99.66425) (width 0.2) (layer "F.Cu") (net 15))
 (segment (start 139.812 96.195649) (end 134.862 101.145649) (width 0.2) (layer "B.Cu") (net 15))
 (segment (start 167.292 99.66425) (end 166.23 98.60225) (width 0.2) (layer "B.Cu") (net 15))
 (segment (start 139.812 95.035851) (end 139.812 96.195649) (width 0.2) (layer "B.Cu") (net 15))
 (segment (start 134.862 101.145649) (end 134.862 117.20575) (width 0.2) (layer "B.Cu") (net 15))
 (segment (start 140.632101 94.21575) (end 139.812 95.035851) (width 0.2) (layer "B.Cu") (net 15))
 (segment (start 141.791899 94.21575) (end 140.632101 94.21575) (width 0.2) (layer "B.Cu") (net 15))
 (segment (start 146.178399 98.60225) (end 141.791899 94.21575) (width 0.2) (layer "B.Cu") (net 15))
 (segment (start 166.23 98.60225) (end 146.178399 98.60225) (width 0.2) (layer "B.Cu") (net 15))
 (segment (start 168.36963 107.28425) (end 174.392 101.26188) (width 0.2) (layer "F.Cu") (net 12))
 (segment (start 174.392 100.098694) (end 176.434944 98.05575) (width 0.2) (layer "F.Cu") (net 12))
 (segment (start 176.434944 98.05575) (end 176.862 98.05575) (width 0.2) (layer "F.Cu") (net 12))
 (segment (start 167.292 107.28425) (end 168.36963 107.28425) (width 0.2) (layer "F.Cu") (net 12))
 (segment (start 174.392 101.26188) (end 174.392 100.098694) (width 0.2) (layer "F.Cu") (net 12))
 (segment (start 176.862 117.10575) (end 170.257143 110.500893) (width 0.2) (layer "F.Cu") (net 13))
 (segment (start 170.257143 110.500893) (end 169.845 110.500893) (width 0.2) (layer "F.Cu") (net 13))
 (via (at 169.845 110.500893) (size 0.6) (drill 0.3) (layers "F.Cu" "B.Cu") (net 13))
 (segment (start 167.292 104.74425) (end 169.845 107.29725) (width 0.2) (layer "B.Cu") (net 13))
 (segment (start 169.845 107.29725) (end 169.845 110.500893) (width 0.2) (layer "B.Cu") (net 13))
 (segment (start 135.002 98.29575) (end 134.862 98.15575) (width 0.2) (layer "F.Cu") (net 14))
 (segment (start 167.484645 98.355) (end 168.355 99.225355) (width 0.2) (layer "B.Cu") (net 14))
 (segment (start 162.188105 93.52225) (end 167.020855 98.355) (width 0.2) (layer "B.Cu") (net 14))
 (segment (start 139.4955 93.52225) (end 162.188105 93.52225) (width 0.2) (layer "B.Cu") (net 14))
 (segment (start 167.020855 98.355) (end 167.484645 98.355) (width 0.2) (layer "B.Cu") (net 14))
 (segment (start 168.355 99.225355) (end 168.355 101.14125) (width 0.2) (layer "B.Cu") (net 14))
 (segment (start 168.355 101.14125) (end 167.292 102.20425) (width 0.2) (layer "B.Cu") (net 14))
 (segment (start 134.862 98.15575) (end 139.4955 93.52225) (width 0.2) (layer "B.Cu") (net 14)))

